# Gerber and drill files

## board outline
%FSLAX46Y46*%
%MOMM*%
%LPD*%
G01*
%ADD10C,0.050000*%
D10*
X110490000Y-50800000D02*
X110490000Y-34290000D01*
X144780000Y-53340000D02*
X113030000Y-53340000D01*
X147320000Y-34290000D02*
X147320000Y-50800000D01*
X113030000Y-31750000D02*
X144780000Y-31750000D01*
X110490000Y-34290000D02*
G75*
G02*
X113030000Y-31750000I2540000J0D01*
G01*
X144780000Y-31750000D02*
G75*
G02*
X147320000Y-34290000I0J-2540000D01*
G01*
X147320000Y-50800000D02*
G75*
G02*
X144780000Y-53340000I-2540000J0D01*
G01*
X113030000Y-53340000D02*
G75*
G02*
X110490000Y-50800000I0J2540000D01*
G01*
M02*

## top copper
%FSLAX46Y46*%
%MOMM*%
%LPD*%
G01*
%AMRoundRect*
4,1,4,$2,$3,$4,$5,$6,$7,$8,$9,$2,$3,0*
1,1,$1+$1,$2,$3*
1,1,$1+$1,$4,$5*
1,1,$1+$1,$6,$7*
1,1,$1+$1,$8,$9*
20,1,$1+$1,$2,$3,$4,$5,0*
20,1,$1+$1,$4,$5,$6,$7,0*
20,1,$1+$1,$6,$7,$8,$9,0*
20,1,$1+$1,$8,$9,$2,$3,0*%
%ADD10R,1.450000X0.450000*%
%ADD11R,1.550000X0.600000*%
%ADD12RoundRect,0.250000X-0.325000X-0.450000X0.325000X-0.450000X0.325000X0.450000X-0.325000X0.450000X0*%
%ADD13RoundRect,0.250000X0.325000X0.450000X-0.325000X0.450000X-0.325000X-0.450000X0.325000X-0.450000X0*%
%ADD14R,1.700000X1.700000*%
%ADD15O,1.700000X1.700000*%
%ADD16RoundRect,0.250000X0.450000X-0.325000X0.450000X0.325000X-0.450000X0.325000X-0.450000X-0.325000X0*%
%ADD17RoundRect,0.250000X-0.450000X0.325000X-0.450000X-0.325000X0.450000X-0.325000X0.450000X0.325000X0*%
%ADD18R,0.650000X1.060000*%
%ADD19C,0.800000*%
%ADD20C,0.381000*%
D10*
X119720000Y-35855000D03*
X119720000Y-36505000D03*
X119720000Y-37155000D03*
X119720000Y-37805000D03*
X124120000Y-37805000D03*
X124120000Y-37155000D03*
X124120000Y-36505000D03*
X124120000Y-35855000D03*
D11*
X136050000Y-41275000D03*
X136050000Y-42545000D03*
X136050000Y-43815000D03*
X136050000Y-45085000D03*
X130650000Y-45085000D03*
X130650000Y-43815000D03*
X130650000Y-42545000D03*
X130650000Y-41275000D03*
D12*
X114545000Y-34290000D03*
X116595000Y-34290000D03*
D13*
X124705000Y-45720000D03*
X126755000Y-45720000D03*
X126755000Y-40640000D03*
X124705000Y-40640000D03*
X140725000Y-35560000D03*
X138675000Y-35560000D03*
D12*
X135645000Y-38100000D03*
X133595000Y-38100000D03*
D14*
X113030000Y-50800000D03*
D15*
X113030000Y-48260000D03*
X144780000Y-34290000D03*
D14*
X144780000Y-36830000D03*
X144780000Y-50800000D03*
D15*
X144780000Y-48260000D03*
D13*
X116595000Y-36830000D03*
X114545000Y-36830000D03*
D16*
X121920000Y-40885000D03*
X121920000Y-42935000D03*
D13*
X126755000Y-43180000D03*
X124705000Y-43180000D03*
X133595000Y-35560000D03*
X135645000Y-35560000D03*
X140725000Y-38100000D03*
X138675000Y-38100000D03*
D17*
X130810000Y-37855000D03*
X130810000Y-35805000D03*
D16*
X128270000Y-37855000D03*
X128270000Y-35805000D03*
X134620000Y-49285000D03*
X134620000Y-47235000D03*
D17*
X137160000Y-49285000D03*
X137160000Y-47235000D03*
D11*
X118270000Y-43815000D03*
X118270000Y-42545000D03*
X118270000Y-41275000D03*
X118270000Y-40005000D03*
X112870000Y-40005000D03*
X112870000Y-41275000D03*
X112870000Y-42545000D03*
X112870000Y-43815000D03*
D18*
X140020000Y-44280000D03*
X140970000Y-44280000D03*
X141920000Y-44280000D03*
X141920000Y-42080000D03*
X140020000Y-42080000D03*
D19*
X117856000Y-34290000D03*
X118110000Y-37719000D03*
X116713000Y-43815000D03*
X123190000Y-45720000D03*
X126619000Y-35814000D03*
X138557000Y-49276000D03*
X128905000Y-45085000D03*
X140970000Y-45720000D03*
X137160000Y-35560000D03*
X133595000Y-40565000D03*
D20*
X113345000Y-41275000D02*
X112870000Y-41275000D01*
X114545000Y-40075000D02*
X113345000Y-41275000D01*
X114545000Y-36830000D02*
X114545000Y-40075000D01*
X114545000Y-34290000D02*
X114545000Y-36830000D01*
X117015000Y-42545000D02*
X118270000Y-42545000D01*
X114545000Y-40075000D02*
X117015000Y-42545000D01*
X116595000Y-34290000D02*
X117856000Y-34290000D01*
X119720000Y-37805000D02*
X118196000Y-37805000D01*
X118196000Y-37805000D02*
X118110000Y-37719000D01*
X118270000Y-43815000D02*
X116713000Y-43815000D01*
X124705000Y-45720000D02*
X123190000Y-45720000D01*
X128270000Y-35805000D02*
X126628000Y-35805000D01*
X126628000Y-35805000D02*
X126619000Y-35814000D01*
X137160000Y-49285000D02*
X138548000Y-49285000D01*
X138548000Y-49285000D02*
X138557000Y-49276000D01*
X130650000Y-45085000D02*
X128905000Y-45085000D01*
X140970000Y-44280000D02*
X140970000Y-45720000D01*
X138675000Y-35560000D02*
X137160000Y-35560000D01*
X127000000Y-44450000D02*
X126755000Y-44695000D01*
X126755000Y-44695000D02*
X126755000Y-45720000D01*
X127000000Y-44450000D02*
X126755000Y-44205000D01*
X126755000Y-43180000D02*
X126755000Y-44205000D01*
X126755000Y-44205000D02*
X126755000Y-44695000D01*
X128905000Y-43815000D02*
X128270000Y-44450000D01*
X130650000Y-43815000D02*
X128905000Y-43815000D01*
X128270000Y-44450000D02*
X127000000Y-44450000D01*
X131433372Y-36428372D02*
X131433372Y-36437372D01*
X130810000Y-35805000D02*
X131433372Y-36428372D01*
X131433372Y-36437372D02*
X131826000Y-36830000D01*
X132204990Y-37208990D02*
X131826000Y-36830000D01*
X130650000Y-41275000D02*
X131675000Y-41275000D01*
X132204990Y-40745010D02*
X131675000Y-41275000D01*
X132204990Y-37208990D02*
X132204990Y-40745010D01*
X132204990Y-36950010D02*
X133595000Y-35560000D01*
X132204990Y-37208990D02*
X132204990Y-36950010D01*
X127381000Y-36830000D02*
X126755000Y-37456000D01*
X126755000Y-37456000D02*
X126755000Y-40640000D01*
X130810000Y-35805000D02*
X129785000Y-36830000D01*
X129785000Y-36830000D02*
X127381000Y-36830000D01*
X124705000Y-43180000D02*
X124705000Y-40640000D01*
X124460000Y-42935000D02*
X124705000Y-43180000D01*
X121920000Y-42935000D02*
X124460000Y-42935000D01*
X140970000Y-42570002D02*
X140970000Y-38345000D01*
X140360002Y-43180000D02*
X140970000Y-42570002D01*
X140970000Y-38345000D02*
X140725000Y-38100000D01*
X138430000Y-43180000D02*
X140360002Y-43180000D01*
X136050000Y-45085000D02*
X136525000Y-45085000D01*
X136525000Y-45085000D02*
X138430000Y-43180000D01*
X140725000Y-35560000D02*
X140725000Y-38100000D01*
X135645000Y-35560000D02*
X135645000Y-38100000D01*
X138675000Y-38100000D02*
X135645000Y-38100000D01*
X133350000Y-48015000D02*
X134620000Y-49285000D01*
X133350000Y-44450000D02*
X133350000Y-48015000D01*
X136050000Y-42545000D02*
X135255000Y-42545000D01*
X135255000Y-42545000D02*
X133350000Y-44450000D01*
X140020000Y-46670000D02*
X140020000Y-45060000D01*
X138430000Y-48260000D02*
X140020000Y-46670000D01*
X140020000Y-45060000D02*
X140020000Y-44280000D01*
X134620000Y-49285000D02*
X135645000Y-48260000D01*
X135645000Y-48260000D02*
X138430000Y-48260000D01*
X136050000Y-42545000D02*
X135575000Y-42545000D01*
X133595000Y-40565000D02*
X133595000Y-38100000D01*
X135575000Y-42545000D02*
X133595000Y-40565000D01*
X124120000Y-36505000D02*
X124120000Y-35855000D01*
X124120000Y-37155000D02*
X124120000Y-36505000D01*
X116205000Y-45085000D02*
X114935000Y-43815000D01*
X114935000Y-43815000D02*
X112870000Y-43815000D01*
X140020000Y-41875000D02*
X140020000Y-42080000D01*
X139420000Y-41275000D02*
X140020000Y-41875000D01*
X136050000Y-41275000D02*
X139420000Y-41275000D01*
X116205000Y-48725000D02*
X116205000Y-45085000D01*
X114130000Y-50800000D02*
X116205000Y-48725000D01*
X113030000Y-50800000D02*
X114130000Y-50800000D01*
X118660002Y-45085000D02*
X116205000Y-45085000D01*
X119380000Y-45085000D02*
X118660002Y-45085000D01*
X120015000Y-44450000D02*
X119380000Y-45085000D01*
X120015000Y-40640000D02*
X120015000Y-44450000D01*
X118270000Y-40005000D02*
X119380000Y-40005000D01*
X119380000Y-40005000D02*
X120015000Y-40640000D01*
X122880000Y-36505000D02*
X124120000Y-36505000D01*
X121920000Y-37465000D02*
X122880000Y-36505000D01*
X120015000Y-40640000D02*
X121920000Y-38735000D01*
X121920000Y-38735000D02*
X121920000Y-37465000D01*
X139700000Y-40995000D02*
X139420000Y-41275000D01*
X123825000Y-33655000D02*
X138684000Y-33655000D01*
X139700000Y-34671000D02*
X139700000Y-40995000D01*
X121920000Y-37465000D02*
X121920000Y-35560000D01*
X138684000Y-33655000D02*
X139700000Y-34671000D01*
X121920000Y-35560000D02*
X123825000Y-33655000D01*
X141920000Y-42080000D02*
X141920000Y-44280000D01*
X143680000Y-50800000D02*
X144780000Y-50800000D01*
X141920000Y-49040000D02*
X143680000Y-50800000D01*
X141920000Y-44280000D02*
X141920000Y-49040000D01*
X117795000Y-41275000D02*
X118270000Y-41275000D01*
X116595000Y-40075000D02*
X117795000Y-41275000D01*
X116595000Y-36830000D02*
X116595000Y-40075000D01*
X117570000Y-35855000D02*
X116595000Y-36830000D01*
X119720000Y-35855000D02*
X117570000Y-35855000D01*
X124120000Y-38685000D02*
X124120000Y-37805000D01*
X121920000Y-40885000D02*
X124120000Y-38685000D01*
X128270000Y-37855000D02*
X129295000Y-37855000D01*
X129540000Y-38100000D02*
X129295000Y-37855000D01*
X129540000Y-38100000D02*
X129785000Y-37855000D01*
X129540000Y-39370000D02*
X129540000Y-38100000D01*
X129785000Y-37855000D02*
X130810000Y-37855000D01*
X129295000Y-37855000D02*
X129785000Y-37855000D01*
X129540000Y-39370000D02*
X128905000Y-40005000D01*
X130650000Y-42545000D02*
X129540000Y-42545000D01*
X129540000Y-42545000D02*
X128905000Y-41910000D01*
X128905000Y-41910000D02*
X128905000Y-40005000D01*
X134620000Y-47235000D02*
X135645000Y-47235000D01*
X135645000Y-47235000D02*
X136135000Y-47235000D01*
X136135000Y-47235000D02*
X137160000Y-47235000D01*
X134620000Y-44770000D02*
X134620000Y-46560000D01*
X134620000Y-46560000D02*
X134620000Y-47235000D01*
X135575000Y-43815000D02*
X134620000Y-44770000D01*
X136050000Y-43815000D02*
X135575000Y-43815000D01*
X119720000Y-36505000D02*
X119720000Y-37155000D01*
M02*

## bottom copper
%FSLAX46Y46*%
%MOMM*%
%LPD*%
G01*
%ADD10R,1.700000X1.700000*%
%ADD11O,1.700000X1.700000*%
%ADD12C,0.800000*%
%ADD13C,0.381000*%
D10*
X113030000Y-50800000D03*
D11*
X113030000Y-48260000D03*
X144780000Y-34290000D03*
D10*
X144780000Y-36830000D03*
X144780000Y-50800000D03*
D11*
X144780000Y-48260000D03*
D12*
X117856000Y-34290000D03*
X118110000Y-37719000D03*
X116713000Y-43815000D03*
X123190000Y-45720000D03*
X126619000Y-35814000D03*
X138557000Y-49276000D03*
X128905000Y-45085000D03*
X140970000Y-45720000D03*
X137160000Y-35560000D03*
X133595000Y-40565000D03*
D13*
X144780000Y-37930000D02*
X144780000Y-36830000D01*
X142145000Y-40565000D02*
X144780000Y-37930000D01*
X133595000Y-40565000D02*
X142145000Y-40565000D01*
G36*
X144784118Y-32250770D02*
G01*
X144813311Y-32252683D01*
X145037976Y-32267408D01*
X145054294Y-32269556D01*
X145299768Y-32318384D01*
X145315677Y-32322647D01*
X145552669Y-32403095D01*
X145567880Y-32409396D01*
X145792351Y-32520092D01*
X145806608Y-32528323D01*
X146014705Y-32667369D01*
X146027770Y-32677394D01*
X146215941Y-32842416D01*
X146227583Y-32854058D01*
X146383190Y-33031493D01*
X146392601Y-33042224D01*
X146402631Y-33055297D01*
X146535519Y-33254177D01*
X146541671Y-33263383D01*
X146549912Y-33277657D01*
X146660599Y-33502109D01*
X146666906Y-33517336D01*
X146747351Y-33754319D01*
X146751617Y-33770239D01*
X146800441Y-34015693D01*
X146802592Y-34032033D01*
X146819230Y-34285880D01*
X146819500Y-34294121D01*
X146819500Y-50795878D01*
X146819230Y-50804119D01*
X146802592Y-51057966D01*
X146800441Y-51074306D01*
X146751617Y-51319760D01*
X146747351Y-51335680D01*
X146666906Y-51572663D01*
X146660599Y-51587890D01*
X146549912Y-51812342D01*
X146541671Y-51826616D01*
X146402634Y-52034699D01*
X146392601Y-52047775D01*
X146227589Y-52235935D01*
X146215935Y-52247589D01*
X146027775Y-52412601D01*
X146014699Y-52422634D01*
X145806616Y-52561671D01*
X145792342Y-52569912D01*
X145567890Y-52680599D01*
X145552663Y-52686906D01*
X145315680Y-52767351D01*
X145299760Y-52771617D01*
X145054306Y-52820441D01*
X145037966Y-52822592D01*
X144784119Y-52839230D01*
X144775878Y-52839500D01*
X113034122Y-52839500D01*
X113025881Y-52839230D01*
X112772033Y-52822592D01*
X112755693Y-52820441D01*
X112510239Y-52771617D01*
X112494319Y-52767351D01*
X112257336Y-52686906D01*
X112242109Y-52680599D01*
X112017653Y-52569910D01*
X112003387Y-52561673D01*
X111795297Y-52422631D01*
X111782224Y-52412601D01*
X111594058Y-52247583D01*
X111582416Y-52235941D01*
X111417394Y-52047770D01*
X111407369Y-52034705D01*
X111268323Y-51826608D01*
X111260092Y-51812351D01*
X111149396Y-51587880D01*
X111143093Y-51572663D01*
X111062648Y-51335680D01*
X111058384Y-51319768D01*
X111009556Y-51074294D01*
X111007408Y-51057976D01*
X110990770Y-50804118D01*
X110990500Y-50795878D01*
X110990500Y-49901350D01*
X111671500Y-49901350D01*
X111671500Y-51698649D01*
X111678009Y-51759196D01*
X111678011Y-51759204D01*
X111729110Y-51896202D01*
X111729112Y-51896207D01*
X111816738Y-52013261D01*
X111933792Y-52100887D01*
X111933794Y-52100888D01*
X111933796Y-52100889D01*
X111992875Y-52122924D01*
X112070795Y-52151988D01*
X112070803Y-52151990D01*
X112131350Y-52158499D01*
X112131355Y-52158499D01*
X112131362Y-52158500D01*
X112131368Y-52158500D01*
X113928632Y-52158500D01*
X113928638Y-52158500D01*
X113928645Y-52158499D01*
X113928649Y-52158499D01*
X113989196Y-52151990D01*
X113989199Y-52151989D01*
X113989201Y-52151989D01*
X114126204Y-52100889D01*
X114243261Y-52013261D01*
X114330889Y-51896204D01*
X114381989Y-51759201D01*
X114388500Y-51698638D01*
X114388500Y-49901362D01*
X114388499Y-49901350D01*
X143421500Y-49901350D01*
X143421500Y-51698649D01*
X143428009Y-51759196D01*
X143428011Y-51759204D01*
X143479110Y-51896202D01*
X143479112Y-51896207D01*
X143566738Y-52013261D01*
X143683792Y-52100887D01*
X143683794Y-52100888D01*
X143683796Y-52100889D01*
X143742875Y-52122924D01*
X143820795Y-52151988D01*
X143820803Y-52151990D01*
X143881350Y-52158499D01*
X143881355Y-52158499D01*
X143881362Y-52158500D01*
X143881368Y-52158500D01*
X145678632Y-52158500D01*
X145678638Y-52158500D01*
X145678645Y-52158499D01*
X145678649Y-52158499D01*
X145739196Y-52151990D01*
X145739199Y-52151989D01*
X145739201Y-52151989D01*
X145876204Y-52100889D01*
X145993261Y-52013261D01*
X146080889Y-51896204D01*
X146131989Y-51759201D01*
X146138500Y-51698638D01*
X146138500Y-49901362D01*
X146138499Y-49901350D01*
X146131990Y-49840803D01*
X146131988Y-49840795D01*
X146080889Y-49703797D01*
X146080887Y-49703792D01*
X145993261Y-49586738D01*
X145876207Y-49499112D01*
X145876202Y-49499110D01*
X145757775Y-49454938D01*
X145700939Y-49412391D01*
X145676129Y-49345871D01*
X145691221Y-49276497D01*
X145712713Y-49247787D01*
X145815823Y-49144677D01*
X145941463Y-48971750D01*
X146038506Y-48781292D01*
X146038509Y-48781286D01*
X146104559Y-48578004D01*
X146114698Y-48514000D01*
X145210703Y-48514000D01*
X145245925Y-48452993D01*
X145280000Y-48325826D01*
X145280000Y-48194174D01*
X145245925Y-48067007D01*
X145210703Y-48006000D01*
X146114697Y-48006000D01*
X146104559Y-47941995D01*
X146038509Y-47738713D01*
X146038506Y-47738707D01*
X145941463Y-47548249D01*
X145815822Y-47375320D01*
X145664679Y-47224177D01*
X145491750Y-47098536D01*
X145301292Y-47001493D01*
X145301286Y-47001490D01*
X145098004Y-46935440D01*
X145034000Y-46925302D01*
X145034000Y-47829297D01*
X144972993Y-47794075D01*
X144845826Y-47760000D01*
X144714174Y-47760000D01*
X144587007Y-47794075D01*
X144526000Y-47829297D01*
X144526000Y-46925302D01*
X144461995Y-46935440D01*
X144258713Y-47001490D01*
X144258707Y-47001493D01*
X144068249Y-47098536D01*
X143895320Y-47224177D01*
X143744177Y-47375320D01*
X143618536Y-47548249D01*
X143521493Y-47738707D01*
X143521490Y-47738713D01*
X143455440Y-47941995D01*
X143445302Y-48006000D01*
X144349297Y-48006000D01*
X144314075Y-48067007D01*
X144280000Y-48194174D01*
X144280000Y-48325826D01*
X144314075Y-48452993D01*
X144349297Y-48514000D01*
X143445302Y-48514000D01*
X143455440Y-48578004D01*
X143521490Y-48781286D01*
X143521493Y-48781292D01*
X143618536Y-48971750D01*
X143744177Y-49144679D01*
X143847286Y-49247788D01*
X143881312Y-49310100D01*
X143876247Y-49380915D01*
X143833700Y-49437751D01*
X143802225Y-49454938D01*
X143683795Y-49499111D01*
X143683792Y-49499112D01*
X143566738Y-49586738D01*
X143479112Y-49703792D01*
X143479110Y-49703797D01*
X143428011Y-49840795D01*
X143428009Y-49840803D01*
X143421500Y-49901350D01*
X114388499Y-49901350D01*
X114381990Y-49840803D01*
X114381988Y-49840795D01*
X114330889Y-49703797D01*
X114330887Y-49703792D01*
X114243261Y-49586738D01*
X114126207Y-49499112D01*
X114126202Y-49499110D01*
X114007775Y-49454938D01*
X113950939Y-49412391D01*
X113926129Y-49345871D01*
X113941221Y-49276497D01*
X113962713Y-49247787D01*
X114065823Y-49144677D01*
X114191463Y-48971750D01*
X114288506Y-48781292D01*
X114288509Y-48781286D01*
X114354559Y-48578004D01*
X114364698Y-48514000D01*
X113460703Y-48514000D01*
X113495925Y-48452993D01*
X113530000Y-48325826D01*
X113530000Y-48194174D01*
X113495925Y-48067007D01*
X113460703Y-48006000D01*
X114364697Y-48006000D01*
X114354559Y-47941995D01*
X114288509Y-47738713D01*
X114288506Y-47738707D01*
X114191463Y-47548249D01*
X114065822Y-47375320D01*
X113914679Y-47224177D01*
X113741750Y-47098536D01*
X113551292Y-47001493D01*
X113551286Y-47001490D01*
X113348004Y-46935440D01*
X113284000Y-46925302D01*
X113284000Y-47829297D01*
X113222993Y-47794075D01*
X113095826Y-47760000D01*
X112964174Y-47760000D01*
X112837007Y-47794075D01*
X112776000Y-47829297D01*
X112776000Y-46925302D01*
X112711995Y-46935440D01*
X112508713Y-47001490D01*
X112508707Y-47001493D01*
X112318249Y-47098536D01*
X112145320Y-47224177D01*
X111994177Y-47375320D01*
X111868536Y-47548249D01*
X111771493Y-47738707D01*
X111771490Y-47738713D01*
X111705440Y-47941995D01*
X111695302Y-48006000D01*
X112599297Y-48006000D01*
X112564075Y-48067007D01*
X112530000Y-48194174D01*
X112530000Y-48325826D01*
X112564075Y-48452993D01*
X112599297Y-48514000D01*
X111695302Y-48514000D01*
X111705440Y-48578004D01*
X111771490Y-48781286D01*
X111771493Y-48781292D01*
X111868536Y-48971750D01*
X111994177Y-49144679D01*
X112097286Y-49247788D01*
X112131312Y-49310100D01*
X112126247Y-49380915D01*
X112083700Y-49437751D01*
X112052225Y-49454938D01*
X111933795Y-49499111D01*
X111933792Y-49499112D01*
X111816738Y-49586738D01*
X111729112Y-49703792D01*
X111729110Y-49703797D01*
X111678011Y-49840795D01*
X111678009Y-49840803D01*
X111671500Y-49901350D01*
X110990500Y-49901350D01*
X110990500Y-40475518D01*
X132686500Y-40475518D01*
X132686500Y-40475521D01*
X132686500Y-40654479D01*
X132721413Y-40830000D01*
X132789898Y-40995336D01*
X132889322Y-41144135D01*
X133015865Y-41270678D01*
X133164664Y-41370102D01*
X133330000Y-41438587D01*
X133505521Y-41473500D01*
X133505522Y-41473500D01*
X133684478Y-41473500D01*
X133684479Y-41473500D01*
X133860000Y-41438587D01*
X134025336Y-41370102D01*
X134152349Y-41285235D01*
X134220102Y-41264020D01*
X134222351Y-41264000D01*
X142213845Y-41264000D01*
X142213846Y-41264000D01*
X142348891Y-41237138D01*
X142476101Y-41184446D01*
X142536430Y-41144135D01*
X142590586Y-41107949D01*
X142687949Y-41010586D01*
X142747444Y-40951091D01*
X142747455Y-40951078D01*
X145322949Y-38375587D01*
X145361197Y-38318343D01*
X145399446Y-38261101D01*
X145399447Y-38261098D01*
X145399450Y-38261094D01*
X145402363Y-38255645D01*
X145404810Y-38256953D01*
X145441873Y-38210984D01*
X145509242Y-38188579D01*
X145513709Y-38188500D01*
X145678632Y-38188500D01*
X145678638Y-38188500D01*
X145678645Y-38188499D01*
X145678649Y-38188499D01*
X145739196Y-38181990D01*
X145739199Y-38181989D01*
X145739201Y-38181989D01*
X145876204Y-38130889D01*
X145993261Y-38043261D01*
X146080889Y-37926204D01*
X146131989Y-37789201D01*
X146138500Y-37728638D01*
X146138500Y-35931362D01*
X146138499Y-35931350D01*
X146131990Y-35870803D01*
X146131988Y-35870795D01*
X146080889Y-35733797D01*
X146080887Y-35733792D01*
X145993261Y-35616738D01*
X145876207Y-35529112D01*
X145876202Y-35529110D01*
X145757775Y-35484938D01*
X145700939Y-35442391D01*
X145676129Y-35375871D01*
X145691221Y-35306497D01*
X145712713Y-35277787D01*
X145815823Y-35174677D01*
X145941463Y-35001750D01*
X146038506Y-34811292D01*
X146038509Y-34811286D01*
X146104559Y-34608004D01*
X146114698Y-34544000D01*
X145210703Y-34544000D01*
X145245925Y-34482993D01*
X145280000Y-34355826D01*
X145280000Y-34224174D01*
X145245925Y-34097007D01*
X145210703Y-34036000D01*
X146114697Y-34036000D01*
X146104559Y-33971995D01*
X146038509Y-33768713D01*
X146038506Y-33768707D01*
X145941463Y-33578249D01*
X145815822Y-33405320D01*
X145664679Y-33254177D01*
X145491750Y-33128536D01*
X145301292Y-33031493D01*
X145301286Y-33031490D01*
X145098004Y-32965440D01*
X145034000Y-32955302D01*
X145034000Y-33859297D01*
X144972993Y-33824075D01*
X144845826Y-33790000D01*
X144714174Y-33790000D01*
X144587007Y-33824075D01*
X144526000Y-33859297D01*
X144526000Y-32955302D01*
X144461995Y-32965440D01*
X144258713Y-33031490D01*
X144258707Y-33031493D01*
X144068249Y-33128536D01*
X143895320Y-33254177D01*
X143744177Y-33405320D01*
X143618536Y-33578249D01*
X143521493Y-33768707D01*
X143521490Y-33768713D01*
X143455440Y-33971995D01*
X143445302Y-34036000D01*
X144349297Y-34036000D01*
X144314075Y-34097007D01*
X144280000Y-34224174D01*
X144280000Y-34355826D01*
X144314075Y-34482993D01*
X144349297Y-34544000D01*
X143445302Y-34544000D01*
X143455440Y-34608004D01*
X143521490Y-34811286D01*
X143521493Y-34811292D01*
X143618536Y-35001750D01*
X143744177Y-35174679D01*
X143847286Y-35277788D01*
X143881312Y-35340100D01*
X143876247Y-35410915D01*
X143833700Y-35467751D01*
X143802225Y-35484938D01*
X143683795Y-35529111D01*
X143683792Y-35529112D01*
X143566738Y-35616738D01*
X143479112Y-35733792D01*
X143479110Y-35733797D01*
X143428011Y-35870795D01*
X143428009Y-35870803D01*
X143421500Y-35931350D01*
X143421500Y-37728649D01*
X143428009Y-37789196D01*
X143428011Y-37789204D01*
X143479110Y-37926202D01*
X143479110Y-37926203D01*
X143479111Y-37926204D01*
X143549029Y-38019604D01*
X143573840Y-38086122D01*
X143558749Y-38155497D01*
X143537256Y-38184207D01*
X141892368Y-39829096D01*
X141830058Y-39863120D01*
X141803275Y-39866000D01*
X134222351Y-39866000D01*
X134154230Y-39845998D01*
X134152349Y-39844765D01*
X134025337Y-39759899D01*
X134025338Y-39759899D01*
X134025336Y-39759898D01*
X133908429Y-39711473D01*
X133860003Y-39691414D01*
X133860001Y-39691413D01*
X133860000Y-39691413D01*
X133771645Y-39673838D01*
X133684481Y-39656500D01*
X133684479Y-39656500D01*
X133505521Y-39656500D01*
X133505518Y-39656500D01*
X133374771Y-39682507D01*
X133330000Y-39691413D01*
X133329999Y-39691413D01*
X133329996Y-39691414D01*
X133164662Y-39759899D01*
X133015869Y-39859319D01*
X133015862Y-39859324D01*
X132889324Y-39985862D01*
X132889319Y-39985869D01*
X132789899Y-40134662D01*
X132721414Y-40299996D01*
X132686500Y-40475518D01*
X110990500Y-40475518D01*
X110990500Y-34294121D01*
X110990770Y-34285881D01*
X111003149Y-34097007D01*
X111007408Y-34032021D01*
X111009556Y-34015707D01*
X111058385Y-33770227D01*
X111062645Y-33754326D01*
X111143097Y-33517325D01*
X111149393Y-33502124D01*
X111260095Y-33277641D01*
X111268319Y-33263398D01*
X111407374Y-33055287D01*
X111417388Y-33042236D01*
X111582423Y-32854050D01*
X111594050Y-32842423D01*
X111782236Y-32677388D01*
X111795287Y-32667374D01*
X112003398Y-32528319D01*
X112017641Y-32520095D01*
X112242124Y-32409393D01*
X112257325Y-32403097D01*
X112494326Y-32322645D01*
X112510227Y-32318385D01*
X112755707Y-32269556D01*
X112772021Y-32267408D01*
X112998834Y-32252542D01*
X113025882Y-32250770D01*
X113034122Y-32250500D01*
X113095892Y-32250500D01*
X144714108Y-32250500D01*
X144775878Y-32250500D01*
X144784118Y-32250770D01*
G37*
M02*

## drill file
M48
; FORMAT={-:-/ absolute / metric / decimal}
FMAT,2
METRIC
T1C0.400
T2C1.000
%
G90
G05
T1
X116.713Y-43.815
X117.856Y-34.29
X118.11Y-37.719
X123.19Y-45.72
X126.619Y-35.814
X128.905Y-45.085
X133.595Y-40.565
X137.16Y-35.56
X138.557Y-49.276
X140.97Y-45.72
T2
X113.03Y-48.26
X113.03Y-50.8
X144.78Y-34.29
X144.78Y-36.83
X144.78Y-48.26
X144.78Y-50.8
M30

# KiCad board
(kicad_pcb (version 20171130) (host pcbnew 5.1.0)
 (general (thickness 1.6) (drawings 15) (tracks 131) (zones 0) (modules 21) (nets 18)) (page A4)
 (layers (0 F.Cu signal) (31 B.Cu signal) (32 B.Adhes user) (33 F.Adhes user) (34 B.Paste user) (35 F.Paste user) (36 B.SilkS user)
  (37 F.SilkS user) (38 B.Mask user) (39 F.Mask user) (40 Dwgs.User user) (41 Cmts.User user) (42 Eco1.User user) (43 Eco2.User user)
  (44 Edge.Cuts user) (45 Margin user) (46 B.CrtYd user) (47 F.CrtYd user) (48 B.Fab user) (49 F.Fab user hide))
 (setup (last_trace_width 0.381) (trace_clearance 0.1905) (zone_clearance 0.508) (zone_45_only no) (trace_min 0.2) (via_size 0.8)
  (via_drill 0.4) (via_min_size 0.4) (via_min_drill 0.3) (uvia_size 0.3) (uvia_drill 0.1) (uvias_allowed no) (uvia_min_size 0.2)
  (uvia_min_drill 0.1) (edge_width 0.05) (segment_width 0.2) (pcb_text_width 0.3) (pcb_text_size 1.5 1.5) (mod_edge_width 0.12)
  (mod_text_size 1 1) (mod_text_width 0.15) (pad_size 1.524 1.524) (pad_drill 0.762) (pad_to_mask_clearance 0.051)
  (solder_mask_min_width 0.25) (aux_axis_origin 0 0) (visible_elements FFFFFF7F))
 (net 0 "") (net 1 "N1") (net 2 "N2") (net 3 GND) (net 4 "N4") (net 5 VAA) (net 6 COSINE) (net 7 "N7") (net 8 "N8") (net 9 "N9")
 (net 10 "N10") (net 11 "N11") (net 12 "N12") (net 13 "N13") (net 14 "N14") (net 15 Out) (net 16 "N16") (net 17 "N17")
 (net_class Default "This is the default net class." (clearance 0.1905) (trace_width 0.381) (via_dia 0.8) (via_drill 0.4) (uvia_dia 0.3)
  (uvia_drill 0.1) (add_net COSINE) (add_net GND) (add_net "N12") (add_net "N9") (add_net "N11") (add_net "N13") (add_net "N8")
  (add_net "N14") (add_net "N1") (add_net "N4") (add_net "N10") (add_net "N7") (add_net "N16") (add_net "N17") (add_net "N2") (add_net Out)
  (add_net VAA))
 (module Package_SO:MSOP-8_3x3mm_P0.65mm (layer F.Cu) (at 121.92 36.83)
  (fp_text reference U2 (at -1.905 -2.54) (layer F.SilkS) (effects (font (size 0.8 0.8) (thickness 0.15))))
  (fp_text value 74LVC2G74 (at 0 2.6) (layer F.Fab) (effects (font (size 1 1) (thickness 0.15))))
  (pad 1 smd rect (at -2.2 -0.975) (size 1.45 0.45) (layers F.Cu F.Paste F.Mask) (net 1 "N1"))
  (pad 2 smd rect (at -2.2 -0.325) (size 1.45 0.45) (layers F.Cu F.Paste F.Mask) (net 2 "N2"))
  (pad 3 smd rect (at -2.2 0.325) (size 1.45 0.45) (layers F.Cu F.Paste F.Mask) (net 2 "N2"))
  (pad 4 smd rect (at -2.2 0.975) (size 1.45 0.45) (layers F.Cu F.Paste F.Mask) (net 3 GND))
  (pad 5 smd rect (at 2.2 0.975) (size 1.45 0.45) (layers F.Cu F.Paste F.Mask) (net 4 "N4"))
  (pad 6 smd rect (at 2.2 0.325) (size 1.45 0.45) (layers F.Cu F.Paste F.Mask) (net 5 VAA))
  (pad 7 smd rect (at 2.2 -0.325) (size 1.45 0.45) (layers F.Cu F.Paste F.Mask) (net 5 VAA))
  (pad 8 smd rect (at 2.2 -0.975) (size 1.45 0.45) (layers F.Cu F.Paste F.Mask) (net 5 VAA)))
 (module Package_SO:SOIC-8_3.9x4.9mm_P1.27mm (layer F.Cu) (at 133.35 43.18)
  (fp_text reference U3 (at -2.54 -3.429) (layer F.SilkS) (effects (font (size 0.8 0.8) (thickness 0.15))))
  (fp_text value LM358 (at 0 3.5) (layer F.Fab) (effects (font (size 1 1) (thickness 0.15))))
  (pad 8 smd rect (at 2.7 -1.905) (size 1.55 0.6) (layers F.Cu F.Paste F.Mask) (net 5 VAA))
  (pad 7 smd rect (at 2.7 -0.635) (size 1.55 0.6) (layers F.Cu F.Paste F.Mask) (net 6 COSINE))
  (pad 6 smd rect (at 2.7 0.635) (size 1.55 0.6) (layers F.Cu F.Paste F.Mask) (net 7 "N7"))
  (pad 5 smd rect (at 2.7 1.905) (size 1.55 0.6) (layers F.Cu F.Paste F.Mask) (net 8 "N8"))
  (pad 4 smd rect (at -2.7 1.905) (size 1.55 0.6) (layers F.Cu F.Paste F.Mask) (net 3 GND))
  (pad 3 smd rect (at -2.7 0.635) (size 1.55 0.6) (layers F.Cu F.Paste F.Mask) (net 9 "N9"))
  (pad 2 smd rect (at -2.7 -0.635) (size 1.55 0.6) (layers F.Cu F.Paste F.Mask) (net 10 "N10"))
  (pad 1 smd rect (at -2.7 -1.905) (size 1.55 0.6) (layers F.Cu F.Paste F.Mask) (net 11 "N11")))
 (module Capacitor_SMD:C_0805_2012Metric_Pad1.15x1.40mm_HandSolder (layer F.Cu) (at 115.57 34.29)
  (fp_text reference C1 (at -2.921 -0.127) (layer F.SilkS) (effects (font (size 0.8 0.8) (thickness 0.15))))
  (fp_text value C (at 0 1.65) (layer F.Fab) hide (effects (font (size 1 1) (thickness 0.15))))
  (pad 1 smd roundrect (at -1.025 0) (size 1.15 1.4) (layers F.Cu F.Paste F.Mask) (roundrect_rratio 0.217391) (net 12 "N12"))
  (pad 2 smd roundrect (at 1.025 0) (size 1.15 1.4) (layers F.Cu F.Paste F.Mask) (roundrect_rratio 0.217391) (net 3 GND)))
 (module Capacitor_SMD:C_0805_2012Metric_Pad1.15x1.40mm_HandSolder (layer F.Cu) (at 125.73 45.72 180)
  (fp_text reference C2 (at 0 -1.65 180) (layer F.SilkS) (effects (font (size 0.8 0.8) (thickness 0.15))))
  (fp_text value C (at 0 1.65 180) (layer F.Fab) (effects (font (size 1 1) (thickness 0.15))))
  (pad 2 smd roundrect (at 1.025 0 180) (size 1.15 1.4) (layers F.Cu F.Paste F.Mask) (roundrect_rratio 0.217391) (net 3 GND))
  (pad 1 smd roundrect (at -1.025 0 180) (size 1.15 1.4) (layers F.Cu F.Paste F.Mask) (roundrect_rratio 0.217391) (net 9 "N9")))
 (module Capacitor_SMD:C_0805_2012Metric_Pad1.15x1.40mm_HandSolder (layer F.Cu) (at 125.73 40.64 180)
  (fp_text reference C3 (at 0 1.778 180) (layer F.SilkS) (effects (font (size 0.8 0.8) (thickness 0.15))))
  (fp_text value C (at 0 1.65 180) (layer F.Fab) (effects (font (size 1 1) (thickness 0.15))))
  (pad 1 smd roundrect (at -1.025 0 180) (size 1.15 1.4) (layers F.Cu F.Paste F.Mask) (roundrect_rratio 0.217391) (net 11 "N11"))
  (pad 2 smd roundrect (at 1.025 0 180) (size 1.15 1.4) (layers F.Cu F.Paste F.Mask) (roundrect_rratio 0.217391) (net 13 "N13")))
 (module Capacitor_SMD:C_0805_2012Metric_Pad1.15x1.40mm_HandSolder (layer F.Cu) (at 139.7 35.56 180)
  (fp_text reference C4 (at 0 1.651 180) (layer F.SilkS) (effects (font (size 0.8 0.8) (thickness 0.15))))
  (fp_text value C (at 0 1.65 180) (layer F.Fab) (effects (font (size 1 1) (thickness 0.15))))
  (pad 1 smd roundrect (at -1.025 0 180) (size 1.15 1.4) (layers F.Cu F.Paste F.Mask) (roundrect_rratio 0.217391) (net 8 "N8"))
  (pad 2 smd roundrect (at 1.025 0 180) (size 1.15 1.4) (layers F.Cu F.Paste F.Mask) (roundrect_rratio 0.217391) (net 3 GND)))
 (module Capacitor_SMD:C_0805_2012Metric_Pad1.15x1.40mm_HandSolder (layer F.Cu) (at 134.62 38.1)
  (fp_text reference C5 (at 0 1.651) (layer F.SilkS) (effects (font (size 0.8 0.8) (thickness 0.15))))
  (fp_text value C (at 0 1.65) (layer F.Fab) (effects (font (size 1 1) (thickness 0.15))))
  (pad 2 smd roundrect (at 1.025 0) (size 1.15 1.4) (layers F.Cu F.Paste F.Mask) (roundrect_rratio 0.217391) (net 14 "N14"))
  (pad 1 smd roundrect (at -1.025 0) (size 1.15 1.4) (layers F.Cu F.Paste F.Mask) (roundrect_rratio 0.217391) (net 6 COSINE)))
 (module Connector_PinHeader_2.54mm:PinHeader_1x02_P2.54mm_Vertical (layer F.Cu) (at 113.03 50.8 180)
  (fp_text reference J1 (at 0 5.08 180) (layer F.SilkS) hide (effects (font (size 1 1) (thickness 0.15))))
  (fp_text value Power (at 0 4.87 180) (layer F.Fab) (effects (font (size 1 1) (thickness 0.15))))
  (pad 1 thru_hole rect (at 0 0 180) (size 1.7 1.7) (drill 1) (layers *.Cu *.Mask) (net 5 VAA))
  (pad 2 thru_hole oval (at 0 2.54 180) (size 1.7 1.7) (drill 1) (layers *.Cu *.Mask) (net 3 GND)))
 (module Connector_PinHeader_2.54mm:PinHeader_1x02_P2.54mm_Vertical (layer F.Cu) (at 144.78 36.83 180)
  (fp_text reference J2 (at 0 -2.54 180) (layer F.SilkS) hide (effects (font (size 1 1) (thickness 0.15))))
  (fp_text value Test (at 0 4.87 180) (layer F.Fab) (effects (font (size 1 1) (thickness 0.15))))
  (pad 2 thru_hole oval (at 0 2.54 180) (size 1.7 1.7) (drill 1) (layers *.Cu *.Mask) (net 3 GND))
  (pad 1 thru_hole rect (at 0 0 180) (size 1.7 1.7) (drill 1) (layers *.Cu *.Mask) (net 6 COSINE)))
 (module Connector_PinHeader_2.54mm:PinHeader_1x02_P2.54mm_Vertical (layer F.Cu) (at 144.78 50.8 180)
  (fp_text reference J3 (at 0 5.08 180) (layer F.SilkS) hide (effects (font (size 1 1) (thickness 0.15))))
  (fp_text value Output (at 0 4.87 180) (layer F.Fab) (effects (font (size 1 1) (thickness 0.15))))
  (pad 1 thru_hole rect (at 0 0 180) (size 1.7 1.7) (drill 1) (layers *.Cu *.Mask) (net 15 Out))
  (pad 2 thru_hole oval (at 0 2.54 180) (size 1.7 1.7) (drill 1) (layers *.Cu *.Mask) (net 3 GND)))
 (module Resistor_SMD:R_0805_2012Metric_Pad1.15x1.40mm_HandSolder (layer F.Cu) (at 115.57 36.83 180)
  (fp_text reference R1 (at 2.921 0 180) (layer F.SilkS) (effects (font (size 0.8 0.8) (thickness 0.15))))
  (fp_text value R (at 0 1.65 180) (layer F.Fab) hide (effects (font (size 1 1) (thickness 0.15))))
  (pad 1 smd roundrect (at -1.025 0 180) (size 1.15 1.4) (layers F.Cu F.Paste F.Mask) (roundrect_rratio 0.217391) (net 1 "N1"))
  (pad 2 smd roundrect (at 1.025 0 180) (size 1.15 1.4) (layers F.Cu F.Paste F.Mask) (roundrect_rratio 0.217391) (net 12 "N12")))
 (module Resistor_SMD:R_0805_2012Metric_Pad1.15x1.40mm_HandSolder (layer F.Cu) (at 121.92 41.91 90)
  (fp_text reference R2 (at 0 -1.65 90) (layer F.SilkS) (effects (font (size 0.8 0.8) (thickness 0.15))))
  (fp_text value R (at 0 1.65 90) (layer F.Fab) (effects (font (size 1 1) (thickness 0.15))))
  (pad 2 smd roundrect (at 1.025 0 90) (size 1.15 1.4) (layers F.Cu F.Paste F.Mask) (roundrect_rratio 0.217391) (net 4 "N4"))
  (pad 1 smd roundrect (at -1.025 0 90) (size 1.15 1.4) (layers F.Cu F.Paste F.Mask) (roundrect_rratio 0.217391) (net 13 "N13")))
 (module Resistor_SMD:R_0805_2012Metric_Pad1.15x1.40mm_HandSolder (layer F.Cu) (at 125.73 43.18 180)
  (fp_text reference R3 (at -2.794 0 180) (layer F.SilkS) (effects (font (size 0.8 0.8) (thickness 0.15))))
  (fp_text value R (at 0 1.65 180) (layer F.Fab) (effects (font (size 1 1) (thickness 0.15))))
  (pad 1 smd roundrect (at -1.025 0 180) (size 1.15 1.4) (layers F.Cu F.Paste F.Mask) (roundrect_rratio 0.217391) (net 9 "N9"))
  (pad 2 smd roundrect (at 1.025 0 180) (size 1.15 1.4) (layers F.Cu F.Paste F.Mask) (roundrect_rratio 0.217391) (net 13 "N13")))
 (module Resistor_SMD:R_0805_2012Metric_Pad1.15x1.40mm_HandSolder (layer F.Cu) (at 134.62 35.56 180)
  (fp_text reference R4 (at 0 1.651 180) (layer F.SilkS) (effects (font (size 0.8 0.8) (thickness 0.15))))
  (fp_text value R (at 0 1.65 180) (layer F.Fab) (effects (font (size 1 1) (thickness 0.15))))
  (pad 2 smd roundrect (at 1.025 0 180) (size 1.15 1.4) (layers F.Cu F.Paste F.Mask) (roundrect_rratio 0.217391) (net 11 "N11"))
  (pad 1 smd roundrect (at -1.025 0 180) (size 1.15 1.4) (layers F.Cu F.Paste F.Mask) (roundrect_rratio 0.217391) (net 14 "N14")))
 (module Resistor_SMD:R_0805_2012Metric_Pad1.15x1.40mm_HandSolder (layer F.Cu) (at 139.7 38.1 180)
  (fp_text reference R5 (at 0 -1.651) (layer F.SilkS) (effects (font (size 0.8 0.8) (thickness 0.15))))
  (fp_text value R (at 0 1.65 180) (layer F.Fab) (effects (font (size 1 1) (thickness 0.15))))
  (pad 1 smd roundrect (at -1.025 0 180) (size 1.15 1.4) (layers F.Cu F.Paste F.Mask) (roundrect_rratio 0.217391) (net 8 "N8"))
  (pad 2 smd roundrect (at 1.025 0 180) (size 1.15 1.4) (layers F.Cu F.Paste F.Mask) (roundrect_rratio 0.217391) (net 14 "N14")))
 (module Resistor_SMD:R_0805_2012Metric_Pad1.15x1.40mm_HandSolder (layer F.Cu) (at 130.81 36.83 270)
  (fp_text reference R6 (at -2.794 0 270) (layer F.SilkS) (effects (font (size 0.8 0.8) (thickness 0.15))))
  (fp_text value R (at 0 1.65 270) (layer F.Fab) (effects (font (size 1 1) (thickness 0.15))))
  (pad 2 smd roundrect (at 1.025 0 270) (size 1.15 1.4) (layers F.Cu F.Paste F.Mask) (roundrect_rratio 0.217391) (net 10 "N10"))
  (pad 1 smd roundrect (at -1.025 0 270) (size 1.15 1.4) (layers F.Cu F.Paste F.Mask) (roundrect_rratio 0.217391) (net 11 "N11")))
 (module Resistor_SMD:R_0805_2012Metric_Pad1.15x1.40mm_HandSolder (layer F.Cu) (at 128.27 36.83 90)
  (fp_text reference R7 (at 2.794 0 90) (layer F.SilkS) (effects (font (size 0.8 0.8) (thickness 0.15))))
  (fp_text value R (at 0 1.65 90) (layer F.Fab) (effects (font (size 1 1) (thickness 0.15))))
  (pad 1 smd roundrect (at -1.025 0 90) (size 1.15 1.4) (layers F.Cu F.Paste F.Mask) (roundrect_rratio 0.217391) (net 10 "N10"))
  (pad 2 smd roundrect (at 1.025 0 90) (size 1.15 1.4) (layers F.Cu F.Paste F.Mask) (roundrect_rratio 0.217391) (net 3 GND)))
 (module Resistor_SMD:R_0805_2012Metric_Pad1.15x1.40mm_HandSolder (layer F.Cu) (at 134.62 48.26 90)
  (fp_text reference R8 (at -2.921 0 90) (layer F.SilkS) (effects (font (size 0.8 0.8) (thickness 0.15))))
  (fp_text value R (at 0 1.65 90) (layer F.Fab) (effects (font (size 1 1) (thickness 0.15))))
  (pad 1 smd roundrect (at -1.025 0 90) (size 1.15 1.4) (layers F.Cu F.Paste F.Mask) (roundrect_rratio 0.217391) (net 6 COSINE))
  (pad 2 smd roundrect (at 1.025 0 90) (size 1.15 1.4) (layers F.Cu F.Paste F.Mask) (roundrect_rratio 0.217391) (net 7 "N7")))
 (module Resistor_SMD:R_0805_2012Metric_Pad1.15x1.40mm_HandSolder (layer F.Cu) (at 137.16 48.26 270)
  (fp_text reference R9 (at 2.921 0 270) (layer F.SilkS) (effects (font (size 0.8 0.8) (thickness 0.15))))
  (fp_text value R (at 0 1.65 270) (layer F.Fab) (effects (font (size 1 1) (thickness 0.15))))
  (pad 2 smd roundrect (at 1.025 0 270) (size 1.15 1.4) (layers F.Cu F.Paste F.Mask) (roundrect_rratio 0.217391) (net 3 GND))
  (pad 1 smd roundrect (at -1.025 0 270) (size 1.15 1.4) (layers F.Cu F.Paste F.Mask) (roundrect_rratio 0.217391) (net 7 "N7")))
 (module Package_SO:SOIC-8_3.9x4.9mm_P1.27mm (layer F.Cu) (at 115.57 41.91 180)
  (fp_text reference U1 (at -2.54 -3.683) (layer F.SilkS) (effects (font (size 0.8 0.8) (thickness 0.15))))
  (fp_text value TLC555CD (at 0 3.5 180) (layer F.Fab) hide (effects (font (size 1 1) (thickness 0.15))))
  (pad 1 smd rect (at -2.7 -1.905 180) (size 1.55 0.6) (layers F.Cu F.Paste F.Mask) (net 3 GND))
  (pad 2 smd rect (at -2.7 -0.635 180) (size 1.55 0.6) (layers F.Cu F.Paste F.Mask) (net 12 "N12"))
  (pad 3 smd rect (at -2.7 0.635 180) (size 1.55 0.6) (layers F.Cu F.Paste F.Mask) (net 1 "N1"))
  (pad 4 smd rect (at -2.7 1.905 180) (size 1.55 0.6) (layers F.Cu F.Paste F.Mask) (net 5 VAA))
  (pad 5 smd rect (at 2.7 1.905 180) (size 1.55 0.6) (layers F.Cu F.Paste F.Mask) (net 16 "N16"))
  (pad 6 smd rect (at 2.7 0.635 180) (size 1.55 0.6) (layers F.Cu F.Paste F.Mask) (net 12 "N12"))
  (pad 7 smd rect (at 2.7 -0.635 180) (size 1.55 0.6) (layers F.Cu F.Paste F.Mask) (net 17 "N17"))
  (pad 8 smd rect (at 2.7 -1.905 180) (size 1.55 0.6) (layers F.Cu F.Paste F.Mask) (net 5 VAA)))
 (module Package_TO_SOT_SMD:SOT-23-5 (layer F.Cu) (at 140.97 43.18 90)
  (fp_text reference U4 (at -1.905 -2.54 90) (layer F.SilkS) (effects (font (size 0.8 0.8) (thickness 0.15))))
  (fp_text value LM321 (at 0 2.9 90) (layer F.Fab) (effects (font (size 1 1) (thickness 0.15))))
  (pad 1 smd rect (at -1.1 -0.95 90) (size 1.06 0.65) (layers F.Cu F.Paste F.Mask) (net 6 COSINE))
  (pad 2 smd rect (at -1.1 0 90) (size 1.06 0.65) (layers F.Cu F.Paste F.Mask) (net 3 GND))
  (pad 3 smd rect (at -1.1 0.95 90) (size 1.06 0.65) (layers F.Cu F.Paste F.Mask) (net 15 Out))
  (pad 4 smd rect (at 1.1 0.95 90) (size 1.06 0.65) (layers F.Cu F.Paste F.Mask) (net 15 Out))
  (pad 5 smd rect (at 1.1 -0.95 90) (size 1.06 0.65) (layers F.Cu F.Paste F.Mask) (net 5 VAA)))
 (gr_line (start 110.49 50.8) (end 110.49 34.29) (layer Edge.Cuts) (width 0.05))
 (gr_line (start 144.78 53.34) (end 113.03 53.34) (layer Edge.Cuts) (width 0.05))
 (gr_line (start 147.32 34.29) (end 147.32 50.8) (layer Edge.Cuts) (width 0.05))
 (gr_line (start 113.03 31.75) (end 144.78 31.75) (layer Edge.Cuts) (width 0.05))
 (gr_arc (start 113.03 34.29) (end 113.03 31.75) (angle -90) (layer Edge.Cuts) (width 0.05))
 (gr_arc (start 144.78 34.29) (end 147.32 34.29) (angle -90) (layer Edge.Cuts) (width 0.05))
 (gr_arc (start 144.78 50.8) (end 144.78 53.34) (angle -90) (layer Edge.Cuts) (width 0.05))
 (gr_arc (start 113.03 50.8) (end 110.49 50.8) (angle -90) (layer Edge.Cuts) (width 0.05))
 (segment (start 113.345 41.275) (end 112.87 41.275) (width 0.381) (layer F.Cu) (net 12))
 (segment (start 114.545 40.075) (end 113.345 41.275) (width 0.381) (layer F.Cu) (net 12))
 (segment (start 114.545 36.83) (end 114.545 40.075) (width 0.381) (layer F.Cu) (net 12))
 (segment (start 114.545 34.29) (end 114.545 36.83) (width 0.381) (layer F.Cu) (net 12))
 (segment (start 117.015 42.545) (end 118.27 42.545) (width 0.381) (layer F.Cu) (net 12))
 (segment (start 114.545 40.075) (end 117.015 42.545) (width 0.381) (layer F.Cu) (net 12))
 (via (at 117.856 34.29) (size 0.8) (drill 0.4) (layers F.Cu B.Cu) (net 3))
 (segment (start 116.595 34.29) (end 117.856 34.29) (width 0.381) (layer F.Cu) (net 3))
 (segment (start 119.72 37.805) (end 118.196 37.805) (width 0.381) (layer F.Cu) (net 3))
 (via (at 118.11 37.719) (size 0.8) (drill 0.4) (layers F.Cu B.Cu) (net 3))
 (segment (start 118.196 37.805) (end 118.11 37.719) (width 0.381) (layer F.Cu) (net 3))
 (via (at 116.713 43.815) (size 0.8) (drill 0.4) (layers F.Cu B.Cu) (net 3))
 (segment (start 118.27 43.815) (end 116.713 43.815) (width 0.381) (layer F.Cu) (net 3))
 (via (at 123.19 45.72) (size 0.8) (drill 0.4) (layers F.Cu B.Cu) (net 3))
 (segment (start 124.705 45.72) (end 123.19 45.72) (width 0.381) (layer F.Cu) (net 3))
 (via (at 126.619 35.814) (size 0.8) (drill 0.4) (layers F.Cu B.Cu) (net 3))
 (segment (start 128.27 35.805) (end 126.628 35.805) (width 0.381) (layer F.Cu) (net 3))
 (segment (start 126.628 35.805) (end 126.619 35.814) (width 0.381) (layer F.Cu) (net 3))
 (via (at 138.557 49.276) (size 0.8) (drill 0.4) (layers F.Cu B.Cu) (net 3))
 (segment (start 137.16 49.285) (end 138.548 49.285) (width 0.381) (layer F.Cu) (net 3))
 (segment (start 138.548 49.285) (end 138.557 49.276) (width 0.381) (layer F.Cu) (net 3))
 (via (at 128.905 45.085) (size 0.8) (drill 0.4) (layers F.Cu B.Cu) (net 3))
 (segment (start 130.65 45.085) (end 128.905 45.085) (width 0.381) (layer F.Cu) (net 3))
 (via (at 140.97 45.72) (size 0.8) (drill 0.4) (layers F.Cu B.Cu) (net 3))
 (segment (start 140.97 44.28) (end 140.97 45.72) (width 0.381) (layer F.Cu) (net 3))
 (via (at 137.16 35.56) (size 0.8) (drill 0.4) (layers F.Cu B.Cu) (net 3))
 (segment (start 138.675 35.56) (end 137.16 35.56) (width 0.381) (layer F.Cu) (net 3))
 (segment (start 127 44.45) (end 126.755 44.695) (width 0.381) (layer F.Cu) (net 9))
 (segment (start 126.755 44.695) (end 126.755 45.72) (width 0.381) (layer F.Cu) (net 9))
 (segment (start 127 44.45) (end 126.755 44.205) (width 0.381) (layer F.Cu) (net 9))
 (segment (start 126.755 43.18) (end 126.755 44.205) (width 0.381) (layer F.Cu) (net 9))
 (segment (start 126.755 44.205) (end 126.755 44.695) (width 0.381) (layer F.Cu) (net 9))
 (segment (start 128.905 43.815) (end 128.27 44.45) (width 0.381) (layer F.Cu) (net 9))
 (segment (start 130.65 43.815) (end 128.905 43.815) (width 0.381) (layer F.Cu) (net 9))
 (segment (start 128.27 44.45) (end 127 44.45) (width 0.381) (layer F.Cu) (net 9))
 (segment (start 131.433372 36.428372) (end 131.433372 36.437372) (width 0.381) (layer F.Cu) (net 11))
 (segment (start 130.81 35.805) (end 131.433372 36.428372) (width 0.381) (layer F.Cu) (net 11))
 (segment (start 131.433372 36.437372) (end 131.826 36.83) (width 0.381) (layer F.Cu) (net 11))
 (segment (start 132.20499 37.20899) (end 131.826 36.83) (width 0.381) (layer F.Cu) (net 11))
 (segment (start 130.65 41.275) (end 131.675 41.275) (width 0.381) (layer F.Cu) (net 11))
 (segment (start 132.20499 40.74501) (end 131.675 41.275) (width 0.381) (layer F.Cu) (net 11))
 (segment (start 132.20499 37.20899) (end 132.20499 40.74501) (width 0.381) (layer F.Cu) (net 11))
 (segment (start 132.20499 36.95001) (end 133.595 35.56) (width 0.381) (layer F.Cu) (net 11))
 (segment (start 132.20499 37.20899) (end 132.20499 36.95001) (width 0.381) (layer F.Cu) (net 11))
 (segment (start 127.381 36.83) (end 126.755 37.456) (width 0.381) (layer F.Cu) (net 11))
 (segment (start 126.755 37.456) (end 126.755 40.64) (width 0.381) (layer F.Cu) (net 11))
 (segment (start 130.81 35.805) (end 129.785 36.83) (width 0.381) (layer F.Cu) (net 11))
 (segment (start 129.785 36.83) (end 127.381 36.83) (width 0.381) (layer F.Cu) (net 11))
 (segment (start 124.705 43.18) (end 124.705 40.64) (width 0.381) (layer F.Cu) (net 13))
 (segment (start 124.46 42.935) (end 124.705 43.18) (width 0.381) (layer F.Cu) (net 13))
 (segment (start 121.92 42.935) (end 124.46 42.935) (width 0.381) (layer F.Cu) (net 13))
 (segment (start 140.97 42.570002) (end 140.97 38.345) (width 0.381) (layer F.Cu) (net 8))
 (segment (start 140.360002 43.18) (end 140.97 42.570002) (width 0.381) (layer F.Cu) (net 8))
 (segment (start 140.97 38.345) (end 140.725 38.1) (width 0.381) (layer F.Cu) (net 8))
 (segment (start 138.43 43.18) (end 140.360002 43.18) (width 0.381) (layer F.Cu) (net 8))
 (segment (start 136.05 45.085) (end 136.525 45.085) (width 0.381) (layer F.Cu) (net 8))
 (segment (start 136.525 45.085) (end 138.43 43.18) (width 0.381) (layer F.Cu) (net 8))
 (segment (start 140.725 35.56) (end 140.725 38.1) (width 0.381) (layer F.Cu) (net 8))
 (segment (start 135.645 35.56) (end 135.645 38.1) (width 0.381) (layer F.Cu) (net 14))
 (segment (start 138.675 38.1) (end 135.645 38.1) (width 0.381) (layer F.Cu) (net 14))
 (segment (start 133.35 48.015) (end 134.62 49.285) (width 0.381) (layer F.Cu) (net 6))
 (segment (start 133.35 44.45) (end 133.35 48.015) (width 0.381) (layer F.Cu) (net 6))
 (segment (start 136.05 42.545) (end 135.255 42.545) (width 0.381) (layer F.Cu) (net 6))
 (segment (start 135.255 42.545) (end 133.35 44.45) (width 0.381) (layer F.Cu) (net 6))
 (segment (start 140.02 46.67) (end 140.02 45.06) (width 0.381) (layer F.Cu) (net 6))
 (segment (start 138.43 48.26) (end 140.02 46.67) (width 0.381) (layer F.Cu) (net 6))
 (segment (start 140.02 45.06) (end 140.02 44.28) (width 0.381) (layer F.Cu) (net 6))
 (segment (start 134.62 49.285) (end 135.645 48.26) (width 0.381) (layer F.Cu) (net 6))
 (segment (start 135.645 48.26) (end 138.43 48.26) (width 0.381) (layer F.Cu) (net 6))
 (segment (start 136.05 42.545) (end 135.575 42.545) (width 0.381) (layer F.Cu) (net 6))
 (segment (start 133.595 40.565) (end 133.595 38.1) (width 0.381) (layer F.Cu) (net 6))
 (segment (start 135.575 42.545) (end 133.595 40.565) (width 0.381) (layer F.Cu) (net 6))
 (via (at 133.595 40.565) (size 0.8) (drill 0.4) (layers F.Cu B.Cu) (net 6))
 (segment (start 144.78 37.93) (end 144.78 36.83) (width 0.381) (layer B.Cu) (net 6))
 (segment (start 142.145 40.565) (end 144.78 37.93) (width 0.381) (layer B.Cu) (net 6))
 (segment (start 133.595 40.565) (end 142.145 40.565) (width 0.381) (layer B.Cu) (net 6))
 (segment (start 124.12 36.505) (end 124.12 35.855) (width 0.381) (layer F.Cu) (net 5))
 (segment (start 124.12 37.155) (end 124.12 36.505) (width 0.381) (layer F.Cu) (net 5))
 (segment (start 116.205 45.085) (end 114.935 43.815) (width 0.381) (layer F.Cu) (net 5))
 (segment (start 114.935 43.815) (end 112.87 43.815) (width 0.381) (layer F.Cu) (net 5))
 (segment (start 140.02 41.875) (end 140.02 42.08) (width 0.381) (layer F.Cu) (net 5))
 (segment (start 139.42 41.275) (end 140.02 41.875) (width 0.381) (layer F.Cu) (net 5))
 (segment (start 136.05 41.275) (end 139.42 41.275) (width 0.381) (layer F.Cu) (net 5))
 (segment (start 116.205 48.725) (end 116.205 45.085) (width 0.381) (layer F.Cu) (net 5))
 (segment (start 114.13 50.8) (end 116.205 48.725) (width 0.381) (layer F.Cu) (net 5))
 (segment (start 113.03 50.8) (end 114.13 50.8) (width 0.381) (layer F.Cu) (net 5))
 (segment (start 118.660002 45.085) (end 116.205 45.085) (width 0.381) (layer F.Cu) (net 5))
 (segment (start 119.38 45.085) (end 118.660002 45.085) (width 0.381) (layer F.Cu) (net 5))
 (segment (start 120.015 44.45) (end 119.38 45.085) (width 0.381) (layer F.Cu) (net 5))
 (segment (start 120.015 40.64) (end 120.015 44.45) (width 0.381) (layer F.Cu) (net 5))
 (segment (start 118.27 40.005) (end 119.38 40.005) (width 0.381) (layer F.Cu) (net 5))
 (segment (start 119.38 40.005) (end 120.015 40.64) (width 0.381) (layer F.Cu) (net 5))
 (segment (start 122.88 36.505) (end 124.12 36.505) (width 0.381) (layer F.Cu) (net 5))
 (segment (start 121.92 37.465) (end 122.88 36.505) (width 0.381) (layer F.Cu) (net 5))
 (segment (start 120.015 40.64) (end 121.92 38.735) (width 0.381) (layer F.Cu) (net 5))
 (segment (start 121.92 38.735) (end 121.92 37.465) (width 0.381) (layer F.Cu) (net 5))
 (segment (start 139.7 40.995) (end 139.42 41.275) (width 0.381) (layer F.Cu) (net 5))
 (segment (start 123.825 33.655) (end 138.684 33.655) (width 0.381) (layer F.Cu) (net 5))
 (segment (start 139.7 34.671) (end 139.7 40.995) (width 0.381) (layer F.Cu) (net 5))
 (segment (start 121.92 37.465) (end 121.92 35.56) (width 0.381) (layer F.Cu) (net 5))
 (segment (start 138.684 33.655) (end 139.7 34.671) (width 0.381) (layer F.Cu) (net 5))
 (segment (start 121.92 35.56) (end 123.825 33.655) (width 0.381) (layer F.Cu) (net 5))
 (segment (start 141.92 42.08) (end 141.92 44.28) (width 0.381) (layer F.Cu) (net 15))
 (segment (start 143.68 50.8) (end 144.78 50.8) (width 0.381) (layer F.Cu) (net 15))
 (segment (start 141.92 49.04) (end 143.68 50.8) (width 0.381) (layer F.Cu) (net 15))
 (segment (start 141.92 44.28) (end 141.92 49.04) (width 0.381) (layer F.Cu) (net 15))
 (segment (start 117.795 41.275) (end 118.27 41.275) (width 0.381) (layer F.Cu) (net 1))
 (segment (start 116.595 40.075) (end 117.795 41.275) (width 0.381) (layer F.Cu) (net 1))
 (segment (start 116.595 36.83) (end 116.595 40.075) (width 0.381) (layer F.Cu) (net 1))
 (segment (start 117.57 35.855) (end 116.595 36.83) (width 0.381) (layer F.Cu) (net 1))
 (segment (start 119.72 35.855) (end 117.57 35.855) (width 0.381) (layer F.Cu) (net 1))
 (segment (start 124.12 38.685) (end 124.12 37.805) (width 0.381) (layer F.Cu) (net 4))
 (segment (start 121.92 40.885) (end 124.12 38.685) (width 0.381) (layer F.Cu) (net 4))
 (segment (start 128.27 37.855) (end 129.295 37.855) (width 0.381) (layer F.Cu) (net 10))
 (segment (start 129.54 38.1) (end 129.295 37.855) (width 0.381) (layer F.Cu) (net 10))
 (segment (start 129.54 38.1) (end 129.785 37.855) (width 0.381) (layer F.Cu) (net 10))
 (segment (start 129.54 39.37) (end 129.54 38.1) (width 0.381) (layer F.Cu) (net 10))
 (segment (start 129.785 37.855) (end 130.81 37.855) (width 0.381) (layer F.Cu) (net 10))
 (segment (start 129.295 37.855) (end 129.785 37.855) (width 0.381) (layer F.Cu) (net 10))
 (segment (start 129.54 39.37) (end 128.905 40.005) (width 0.381) (layer F.Cu) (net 10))
 (segment (start 130.65 42.545) (end 129.54 42.545) (width 0.381) (layer F.Cu) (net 10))
 (segment (start 129.54 42.545) (end 128.905 41.91) (width 0.381) (layer F.Cu) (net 10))
 (segment (start 128.905 41.91) (end 128.905 40.005) (width 0.381) (layer F.Cu) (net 10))
 (segment (start 134.62 47.235) (end 135.645 47.235) (width 0.381) (layer F.Cu) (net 7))
 (segment (start 135.645 47.235) (end 136.135 47.235) (width 0.381) (layer F.Cu) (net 7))
 (segment (start 136.135 47.235) (end 137.16 47.235) (width 0.381) (layer F.Cu) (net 7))
 (segment (start 134.62 44.77) (end 134.62 46.56) (width 0.381) (layer F.Cu) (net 7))
 (segment (start 134.62 46.56) (end 134.62 47.235) (width 0.381) (layer F.Cu) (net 7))
 (segment (start 135.575 43.815) (end 134.62 44.77) (width 0.381) (layer F.Cu) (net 7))
 (segment (start 136.05 43.815) (end 135.575 43.815) (width 0.381) (layer F.Cu) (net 7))
 (segment (start 119.72 36.505) (end 119.72 37.155) (width 0.381) (layer F.Cu) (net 2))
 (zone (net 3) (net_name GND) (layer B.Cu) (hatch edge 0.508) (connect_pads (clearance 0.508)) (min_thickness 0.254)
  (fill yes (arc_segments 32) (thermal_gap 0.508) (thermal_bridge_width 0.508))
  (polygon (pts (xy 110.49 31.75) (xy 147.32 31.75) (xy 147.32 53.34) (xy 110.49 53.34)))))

